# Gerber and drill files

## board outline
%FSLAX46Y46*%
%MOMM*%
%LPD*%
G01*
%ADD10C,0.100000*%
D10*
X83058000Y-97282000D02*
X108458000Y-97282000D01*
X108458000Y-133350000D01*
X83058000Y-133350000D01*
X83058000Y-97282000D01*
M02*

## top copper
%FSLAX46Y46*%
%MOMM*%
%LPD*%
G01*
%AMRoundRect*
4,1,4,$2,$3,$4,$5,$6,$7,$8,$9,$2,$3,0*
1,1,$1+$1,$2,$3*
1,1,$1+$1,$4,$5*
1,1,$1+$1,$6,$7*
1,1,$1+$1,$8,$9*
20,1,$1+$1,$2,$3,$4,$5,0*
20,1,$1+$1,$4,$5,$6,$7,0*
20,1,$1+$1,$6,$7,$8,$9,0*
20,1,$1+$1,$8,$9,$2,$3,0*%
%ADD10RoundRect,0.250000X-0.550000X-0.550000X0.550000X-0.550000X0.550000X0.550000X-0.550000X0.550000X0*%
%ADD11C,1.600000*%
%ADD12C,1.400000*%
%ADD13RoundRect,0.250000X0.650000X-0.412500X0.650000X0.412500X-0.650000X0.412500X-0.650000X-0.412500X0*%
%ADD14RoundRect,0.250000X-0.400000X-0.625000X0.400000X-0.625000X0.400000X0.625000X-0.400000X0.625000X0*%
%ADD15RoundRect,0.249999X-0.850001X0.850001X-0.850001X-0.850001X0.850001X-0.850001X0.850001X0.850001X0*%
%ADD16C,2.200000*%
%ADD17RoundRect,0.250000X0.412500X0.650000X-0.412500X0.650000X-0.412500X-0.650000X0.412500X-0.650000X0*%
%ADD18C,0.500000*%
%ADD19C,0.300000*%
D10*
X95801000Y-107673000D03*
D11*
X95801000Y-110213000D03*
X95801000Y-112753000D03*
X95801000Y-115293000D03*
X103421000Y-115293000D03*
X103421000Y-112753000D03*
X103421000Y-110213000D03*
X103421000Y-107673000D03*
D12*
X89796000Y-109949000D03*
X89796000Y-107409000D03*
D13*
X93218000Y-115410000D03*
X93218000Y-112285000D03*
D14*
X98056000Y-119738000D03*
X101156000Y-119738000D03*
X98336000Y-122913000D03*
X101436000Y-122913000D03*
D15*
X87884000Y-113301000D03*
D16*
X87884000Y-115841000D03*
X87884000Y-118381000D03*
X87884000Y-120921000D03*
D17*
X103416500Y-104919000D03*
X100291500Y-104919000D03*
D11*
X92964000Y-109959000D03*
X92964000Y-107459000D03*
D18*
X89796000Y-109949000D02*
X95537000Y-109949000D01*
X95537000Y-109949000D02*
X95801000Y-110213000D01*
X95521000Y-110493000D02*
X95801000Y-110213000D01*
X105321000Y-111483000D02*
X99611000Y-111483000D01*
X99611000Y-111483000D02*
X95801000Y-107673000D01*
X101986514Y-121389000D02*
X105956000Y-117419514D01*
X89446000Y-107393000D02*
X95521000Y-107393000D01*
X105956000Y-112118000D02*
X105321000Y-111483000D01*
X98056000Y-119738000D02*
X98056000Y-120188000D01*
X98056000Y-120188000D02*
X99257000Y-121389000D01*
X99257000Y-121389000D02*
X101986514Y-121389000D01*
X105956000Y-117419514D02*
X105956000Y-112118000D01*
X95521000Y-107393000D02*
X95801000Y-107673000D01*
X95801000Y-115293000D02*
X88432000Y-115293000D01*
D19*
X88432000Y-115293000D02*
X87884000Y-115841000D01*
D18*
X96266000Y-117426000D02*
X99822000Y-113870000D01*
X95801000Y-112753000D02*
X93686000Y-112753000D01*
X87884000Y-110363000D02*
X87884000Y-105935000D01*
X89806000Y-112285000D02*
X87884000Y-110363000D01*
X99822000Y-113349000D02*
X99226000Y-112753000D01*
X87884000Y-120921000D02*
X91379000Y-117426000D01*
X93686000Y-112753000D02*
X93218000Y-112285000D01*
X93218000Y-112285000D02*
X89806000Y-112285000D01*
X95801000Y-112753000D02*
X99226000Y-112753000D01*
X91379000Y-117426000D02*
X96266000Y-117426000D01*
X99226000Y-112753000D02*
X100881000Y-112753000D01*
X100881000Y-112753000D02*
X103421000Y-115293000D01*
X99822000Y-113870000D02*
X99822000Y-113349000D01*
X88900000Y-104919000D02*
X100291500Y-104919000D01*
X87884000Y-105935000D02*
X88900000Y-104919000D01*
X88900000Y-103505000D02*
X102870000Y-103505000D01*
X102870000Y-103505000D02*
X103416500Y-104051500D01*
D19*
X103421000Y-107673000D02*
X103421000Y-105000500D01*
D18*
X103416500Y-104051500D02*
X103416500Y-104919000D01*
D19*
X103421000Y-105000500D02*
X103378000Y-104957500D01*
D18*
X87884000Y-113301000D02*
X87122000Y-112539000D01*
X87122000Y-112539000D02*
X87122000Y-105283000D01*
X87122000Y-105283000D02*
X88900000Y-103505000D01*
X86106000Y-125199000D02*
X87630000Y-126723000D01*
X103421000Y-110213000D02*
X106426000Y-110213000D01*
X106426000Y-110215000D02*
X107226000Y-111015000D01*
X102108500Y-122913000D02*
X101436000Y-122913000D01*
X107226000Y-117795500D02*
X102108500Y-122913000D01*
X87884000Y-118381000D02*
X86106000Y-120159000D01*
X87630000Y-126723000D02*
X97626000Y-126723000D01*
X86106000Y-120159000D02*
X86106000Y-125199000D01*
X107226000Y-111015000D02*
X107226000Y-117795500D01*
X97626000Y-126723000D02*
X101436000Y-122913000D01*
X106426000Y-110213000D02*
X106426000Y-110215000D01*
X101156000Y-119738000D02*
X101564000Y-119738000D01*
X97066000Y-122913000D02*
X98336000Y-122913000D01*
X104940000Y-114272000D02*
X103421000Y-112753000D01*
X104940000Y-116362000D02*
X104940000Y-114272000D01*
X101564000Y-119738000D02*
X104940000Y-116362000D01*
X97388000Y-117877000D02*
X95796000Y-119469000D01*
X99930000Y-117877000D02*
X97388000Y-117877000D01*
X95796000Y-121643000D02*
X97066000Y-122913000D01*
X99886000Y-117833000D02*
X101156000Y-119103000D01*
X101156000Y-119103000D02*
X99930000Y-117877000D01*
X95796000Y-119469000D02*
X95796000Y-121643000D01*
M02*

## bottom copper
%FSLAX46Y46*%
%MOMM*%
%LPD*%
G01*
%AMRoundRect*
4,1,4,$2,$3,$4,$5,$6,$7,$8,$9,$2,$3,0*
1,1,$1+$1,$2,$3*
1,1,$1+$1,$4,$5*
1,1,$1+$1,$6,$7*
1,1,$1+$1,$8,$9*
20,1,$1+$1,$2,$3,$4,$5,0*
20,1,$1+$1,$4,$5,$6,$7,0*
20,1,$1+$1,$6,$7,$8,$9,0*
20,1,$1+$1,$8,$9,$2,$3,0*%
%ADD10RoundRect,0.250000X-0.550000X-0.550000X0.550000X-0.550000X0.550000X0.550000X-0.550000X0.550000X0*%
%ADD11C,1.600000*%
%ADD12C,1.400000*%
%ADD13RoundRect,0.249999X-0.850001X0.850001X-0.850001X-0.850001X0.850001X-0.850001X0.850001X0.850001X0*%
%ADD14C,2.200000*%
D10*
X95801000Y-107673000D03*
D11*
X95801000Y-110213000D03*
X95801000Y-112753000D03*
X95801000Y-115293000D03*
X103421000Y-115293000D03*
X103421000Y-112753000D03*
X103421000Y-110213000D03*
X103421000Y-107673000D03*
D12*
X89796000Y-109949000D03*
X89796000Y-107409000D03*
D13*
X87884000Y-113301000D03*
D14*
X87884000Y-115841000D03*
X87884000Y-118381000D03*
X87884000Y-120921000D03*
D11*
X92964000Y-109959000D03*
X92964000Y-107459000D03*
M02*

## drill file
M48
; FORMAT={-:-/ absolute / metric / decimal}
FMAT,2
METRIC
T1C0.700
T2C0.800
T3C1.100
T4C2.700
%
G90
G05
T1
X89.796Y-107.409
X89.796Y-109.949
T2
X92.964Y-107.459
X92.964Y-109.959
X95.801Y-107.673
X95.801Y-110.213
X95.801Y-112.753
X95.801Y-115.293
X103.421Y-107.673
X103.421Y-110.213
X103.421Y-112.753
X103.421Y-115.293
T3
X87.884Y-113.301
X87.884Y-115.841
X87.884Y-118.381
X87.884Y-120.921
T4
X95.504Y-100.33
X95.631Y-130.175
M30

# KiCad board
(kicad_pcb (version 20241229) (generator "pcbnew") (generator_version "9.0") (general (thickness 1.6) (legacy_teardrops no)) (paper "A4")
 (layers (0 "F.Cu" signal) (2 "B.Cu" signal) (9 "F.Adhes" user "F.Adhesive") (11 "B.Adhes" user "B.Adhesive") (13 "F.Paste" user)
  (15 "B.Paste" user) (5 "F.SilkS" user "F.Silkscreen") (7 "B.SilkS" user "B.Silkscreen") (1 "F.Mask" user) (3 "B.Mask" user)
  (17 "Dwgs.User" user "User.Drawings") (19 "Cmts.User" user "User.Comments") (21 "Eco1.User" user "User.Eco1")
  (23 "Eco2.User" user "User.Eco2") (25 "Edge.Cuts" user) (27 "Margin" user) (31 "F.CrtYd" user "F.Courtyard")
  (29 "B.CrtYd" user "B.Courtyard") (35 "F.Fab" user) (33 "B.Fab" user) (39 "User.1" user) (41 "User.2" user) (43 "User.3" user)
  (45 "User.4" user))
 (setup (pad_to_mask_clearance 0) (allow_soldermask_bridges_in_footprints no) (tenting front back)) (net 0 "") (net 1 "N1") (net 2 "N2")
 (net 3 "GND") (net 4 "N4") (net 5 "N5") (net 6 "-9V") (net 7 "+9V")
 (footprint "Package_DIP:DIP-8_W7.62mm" (layer "F.Cu") (at 95.801 107.673)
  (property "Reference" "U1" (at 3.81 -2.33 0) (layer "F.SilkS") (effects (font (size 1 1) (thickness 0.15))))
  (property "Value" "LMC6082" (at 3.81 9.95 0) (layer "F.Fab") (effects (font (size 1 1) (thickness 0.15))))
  (pad "1" thru_hole roundrect (at 0 0) (size 1.6 1.6) (drill 0.8) (layers "*.Cu" "*.Mask") (remove_unused_layers no)
   (roundrect_rratio 0.15625) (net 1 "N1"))
  (pad "2" thru_hole circle (at 0 2.54) (size 1.6 1.6) (drill 0.8) (layers "*.Cu" "*.Mask") (remove_unused_layers no) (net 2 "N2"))
  (pad "3" thru_hole circle (at 0 5.08) (size 1.6 1.6) (drill 0.8) (layers "*.Cu" "*.Mask") (remove_unused_layers no) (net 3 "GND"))
  (pad "4" thru_hole circle (at 0 7.62) (size 1.6 1.6) (drill 0.8) (layers "*.Cu" "*.Mask") (remove_unused_layers no))
  (pad "5" thru_hole circle (at 7.62 7.62) (size 1.6 1.6) (drill 0.8) (layers "*.Cu" "*.Mask") (remove_unused_layers no) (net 3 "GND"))
  (pad "6" thru_hole circle (at 7.62 5.08) (size 1.6 1.6) (drill 0.8) (layers "*.Cu" "*.Mask") (remove_unused_layers no) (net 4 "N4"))
  (pad "7" thru_hole circle (at 7.62 2.54) (size 1.6 1.6) (drill 0.8) (layers "*.Cu" "*.Mask") (remove_unused_layers no) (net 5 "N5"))
  (pad "8" thru_hole circle (at 7.62 0) (size 1.6 1.6) (drill 0.8) (layers "*.Cu" "*.Mask") (remove_unused_layers no)))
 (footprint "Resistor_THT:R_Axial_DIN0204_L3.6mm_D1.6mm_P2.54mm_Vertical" (layer "F.Cu") (at 89.796 109.949 90)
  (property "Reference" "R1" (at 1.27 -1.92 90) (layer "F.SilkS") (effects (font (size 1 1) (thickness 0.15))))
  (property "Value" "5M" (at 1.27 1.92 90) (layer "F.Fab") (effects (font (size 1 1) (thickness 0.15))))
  (pad "1" thru_hole circle (at 0 0 90) (size 1.4 1.4) (drill 0.7) (layers "*.Cu" "*.Mask") (remove_unused_layers no) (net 2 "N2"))
  (pad "2" thru_hole circle (at 2.54 0 90) (size 1.4 1.4) (drill 0.7) (layers "*.Cu" "*.Mask") (remove_unused_layers no) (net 1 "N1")))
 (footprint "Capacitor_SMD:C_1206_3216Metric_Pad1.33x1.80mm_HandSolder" (layer "F.Cu") (at 93.218 113.8475 90)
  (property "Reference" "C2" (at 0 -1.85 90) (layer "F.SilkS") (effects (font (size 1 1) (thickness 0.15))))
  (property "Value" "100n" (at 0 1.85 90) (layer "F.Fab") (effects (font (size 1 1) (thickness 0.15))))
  (pad "1" smd roundrect (at -1.5625 0 90) (size 1.325 1.8) (layers "F.Cu" "F.Mask" "F.Paste") (roundrect_rratio 0.188679) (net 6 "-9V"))
  (pad "2" smd roundrect (at 1.5625 0 90) (size 1.325 1.8) (layers "F.Cu" "F.Mask" "F.Paste") (roundrect_rratio 0.188679) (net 3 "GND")))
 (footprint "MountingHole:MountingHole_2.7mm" (layer "F.Cu") (at 95.631 130.175)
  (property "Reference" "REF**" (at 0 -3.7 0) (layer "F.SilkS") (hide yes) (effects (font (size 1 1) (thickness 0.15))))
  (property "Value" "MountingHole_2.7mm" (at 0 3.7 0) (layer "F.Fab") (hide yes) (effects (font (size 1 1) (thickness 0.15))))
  (pad "" np_thru_hole circle (at 0 0) (size 2.7 2.7) (drill 2.7) (layers "*.Cu" "*.Mask")))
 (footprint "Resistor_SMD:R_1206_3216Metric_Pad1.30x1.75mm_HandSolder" (layer "F.Cu") (at 99.606 119.738)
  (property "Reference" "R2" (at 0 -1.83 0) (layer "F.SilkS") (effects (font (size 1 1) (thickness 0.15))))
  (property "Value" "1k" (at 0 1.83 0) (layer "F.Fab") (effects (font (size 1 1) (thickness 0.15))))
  (pad "1" smd roundrect (at -1.55 0) (size 1.3 1.75) (layers "F.Cu" "F.Mask" "F.Paste") (roundrect_rratio 0.192308) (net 1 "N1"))
  (pad "2" smd roundrect (at 1.55 0) (size 1.3 1.75) (layers "F.Cu" "F.Mask" "F.Paste") (roundrect_rratio 0.192308) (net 4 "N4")))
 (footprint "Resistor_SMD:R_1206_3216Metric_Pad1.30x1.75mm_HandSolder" (layer "F.Cu") (at 99.886 122.913)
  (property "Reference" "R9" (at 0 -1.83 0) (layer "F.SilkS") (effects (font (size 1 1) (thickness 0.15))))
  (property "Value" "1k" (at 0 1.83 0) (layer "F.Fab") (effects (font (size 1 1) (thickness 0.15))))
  (pad "1" smd roundrect (at -1.55 0) (size 1.3 1.75) (layers "F.Cu" "F.Mask" "F.Paste") (roundrect_rratio 0.192308) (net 4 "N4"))
  (pad "2" smd roundrect (at 1.55 0) (size 1.3 1.75) (layers "F.Cu" "F.Mask" "F.Paste") (roundrect_rratio 0.192308) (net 5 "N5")))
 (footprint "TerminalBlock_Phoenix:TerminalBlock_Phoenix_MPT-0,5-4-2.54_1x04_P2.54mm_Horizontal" (layer "F.Cu") (at 87.884 113.301 -90)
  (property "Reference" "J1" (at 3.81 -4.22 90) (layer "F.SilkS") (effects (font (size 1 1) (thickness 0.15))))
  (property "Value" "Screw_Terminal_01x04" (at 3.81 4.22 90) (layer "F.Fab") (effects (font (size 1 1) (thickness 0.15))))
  (pad "1" thru_hole roundrect (at 0 0 270) (size 2.2 2.2) (drill 1.1) (layers "*.Cu" "*.Mask") (remove_unused_layers no)
   (roundrect_rratio 0.113636) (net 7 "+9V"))
  (pad "2" thru_hole circle (at 2.54 0 270) (size 2.2 2.2) (drill 1.1) (layers "*.Cu" "*.Mask") (remove_unused_layers no) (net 6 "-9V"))
  (pad "3" thru_hole circle (at 5.08 0 270) (size 2.2 2.2) (drill 1.1) (layers "*.Cu" "*.Mask") (remove_unused_layers no) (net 5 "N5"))
  (pad "4" thru_hole circle (at 7.62 0 270) (size 2.2 2.2) (drill 1.1) (layers "*.Cu" "*.Mask") (remove_unused_layers no) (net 3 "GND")))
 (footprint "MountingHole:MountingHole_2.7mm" (layer "F.Cu") (at 95.504 100.33)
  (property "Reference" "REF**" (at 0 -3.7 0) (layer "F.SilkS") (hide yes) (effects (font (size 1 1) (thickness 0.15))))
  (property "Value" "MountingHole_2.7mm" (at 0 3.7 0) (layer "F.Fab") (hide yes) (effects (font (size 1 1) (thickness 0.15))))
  (pad "" np_thru_hole circle (at 0 0) (size 2.7 2.7) (drill 2.7) (layers "*.Cu" "*.Mask")))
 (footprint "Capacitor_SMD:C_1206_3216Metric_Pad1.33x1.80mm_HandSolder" (layer "F.Cu") (at 101.854 104.919 180)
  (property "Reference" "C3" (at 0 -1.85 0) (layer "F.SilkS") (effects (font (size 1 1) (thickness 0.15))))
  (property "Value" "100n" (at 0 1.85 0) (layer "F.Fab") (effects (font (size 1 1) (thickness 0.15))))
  (pad "1" smd roundrect (at -1.5625 0 180) (size 1.325 1.8) (layers "F.Cu" "F.Mask" "F.Paste") (roundrect_rratio 0.188679) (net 7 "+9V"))
  (pad "2" smd roundrect (at 1.5625 0 180) (size 1.325 1.8) (layers "F.Cu" "F.Mask" "F.Paste") (roundrect_rratio 0.188679) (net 3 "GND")))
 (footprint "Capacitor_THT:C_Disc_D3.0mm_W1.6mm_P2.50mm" (layer "F.Cu") (at 92.964 109.959 90)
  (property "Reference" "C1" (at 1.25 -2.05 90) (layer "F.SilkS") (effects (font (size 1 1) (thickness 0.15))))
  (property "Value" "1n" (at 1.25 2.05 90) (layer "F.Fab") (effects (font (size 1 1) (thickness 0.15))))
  (pad "1" thru_hole circle (at 0 0 90) (size 1.6 1.6) (drill 0.8) (layers "*.Cu" "*.Mask") (remove_unused_layers no) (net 2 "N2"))
  (pad "2" thru_hole circle (at 2.5 0 90) (size 1.6 1.6) (drill 0.8) (layers "*.Cu" "*.Mask") (remove_unused_layers no) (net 1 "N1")))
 (gr_rect (start 83.058 97.282) (end 108.458 133.35) (stroke (width 0.1) (type solid)) (fill no) (layer "Edge.Cuts"))
 (segment (start 89.796 109.949) (end 95.537 109.949) (width 0.5) (layer "F.Cu") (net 2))
 (segment (start 95.537 109.949) (end 95.801 110.213) (width 0.5) (layer "F.Cu") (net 2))
 (segment (start 95.521 110.493) (end 95.801 110.213) (width 0.5) (layer "F.Cu") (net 2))
 (segment (start 105.321 111.483) (end 99.611 111.483) (width 0.5) (layer "F.Cu") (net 1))
 (segment (start 99.611 111.483) (end 95.801 107.673) (width 0.5) (layer "F.Cu") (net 1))
 (segment (start 101.986514 121.389) (end 105.956 117.419514) (width 0.5) (layer "F.Cu") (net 1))
 (segment (start 89.446 107.393) (end 95.521 107.393) (width 0.5) (layer "F.Cu") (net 1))
 (segment (start 105.956 112.118) (end 105.321 111.483) (width 0.5) (layer "F.Cu") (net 1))
 (segment (start 98.056 119.738) (end 98.056 120.188) (width 0.5) (layer "F.Cu") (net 1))
 (segment (start 98.056 120.188) (end 99.257 121.389) (width 0.5) (layer "F.Cu") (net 1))
 (segment (start 99.257 121.389) (end 101.986514 121.389) (width 0.5) (layer "F.Cu") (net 1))
 (segment (start 105.956 117.419514) (end 105.956 112.118) (width 0.5) (layer "F.Cu") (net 1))
 (segment (start 95.521 107.393) (end 95.801 107.673) (width 0.5) (layer "F.Cu") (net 1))
 (segment (start 95.801 115.293) (end 88.432 115.293) (width 0.5) (layer "F.Cu") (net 6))
 (segment (start 88.432 115.293) (end 87.884 115.841) (width 0.3) (layer "F.Cu") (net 6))
 (segment (start 96.266 117.426) (end 99.822 113.87) (width 0.5) (layer "F.Cu") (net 3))
 (segment (start 95.801 112.753) (end 93.686 112.753) (width 0.5) (layer "F.Cu") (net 3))
 (segment (start 87.884 110.363) (end 87.884 105.935) (width 0.5) (layer "F.Cu") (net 3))
 (segment (start 89.806 112.285) (end 87.884 110.363) (width 0.5) (layer "F.Cu") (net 3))
 (segment (start 99.822 113.349) (end 99.226 112.753) (width 0.5) (layer "F.Cu") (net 3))
 (segment (start 87.884 120.921) (end 91.379 117.426) (width 0.5) (layer "F.Cu") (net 3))
 (segment (start 93.686 112.753) (end 93.218 112.285) (width 0.5) (layer "F.Cu") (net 3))
 (segment (start 93.218 112.285) (end 89.806 112.285) (width 0.5) (layer "F.Cu") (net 3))
 (segment (start 95.801 112.753) (end 99.226 112.753) (width 0.5) (layer "F.Cu") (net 3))
 (segment (start 91.379 117.426) (end 96.266 117.426) (width 0.5) (layer "F.Cu") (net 3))
 (segment (start 99.226 112.753) (end 100.881 112.753) (width 0.5) (layer "F.Cu") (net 3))
 (segment (start 100.881 112.753) (end 103.421 115.293) (width 0.5) (layer "F.Cu") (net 3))
 (segment (start 99.822 113.87) (end 99.822 113.349) (width 0.5) (layer "F.Cu") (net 3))
 (segment (start 88.9 104.919) (end 100.2915 104.919) (width 0.5) (layer "F.Cu") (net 3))
 (segment (start 87.884 105.935) (end 88.9 104.919) (width 0.5) (layer "F.Cu") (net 3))
 (segment (start 88.9 103.505) (end 102.87 103.505) (width 0.5) (layer "F.Cu") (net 7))
 (segment (start 102.87 103.505) (end 103.4165 104.0515) (width 0.5) (layer "F.Cu") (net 7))
 (segment (start 103.421 107.673) (end 103.421 105.0005) (width 0.3) (layer "F.Cu") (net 7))
 (segment (start 103.4165 104.0515) (end 103.4165 104.919) (width 0.5) (layer "F.Cu") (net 7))
 (segment (start 103.421 105.0005) (end 103.378 104.9575) (width 0.3) (layer "F.Cu") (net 7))
 (segment (start 87.884 113.301) (end 87.122 112.539) (width 0.5) (layer "F.Cu") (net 7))
 (segment (start 87.122 112.539) (end 87.122 105.283) (width 0.5) (layer "F.Cu") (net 7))
 (segment (start 87.122 105.283) (end 88.9 103.505) (width 0.5) (layer "F.Cu") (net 7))
 (segment (start 86.106 125.199) (end 87.63 126.723) (width 0.5) (layer "F.Cu") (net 5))
 (segment (start 103.421 110.213) (end 106.426 110.213) (width 0.5) (layer "F.Cu") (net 5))
 (segment (start 106.426 110.215) (end 107.226 111.015) (width 0.5) (layer "F.Cu") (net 5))
 (segment (start 102.1085 122.913) (end 101.436 122.913) (width 0.5) (layer "F.Cu") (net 5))
 (segment (start 107.226 117.7955) (end 102.1085 122.913) (width 0.5) (layer "F.Cu") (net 5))
 (segment (start 87.884 118.381) (end 86.106 120.159) (width 0.5) (layer "F.Cu") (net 5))
 (segment (start 87.63 126.723) (end 97.626 126.723) (width 0.5) (layer "F.Cu") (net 5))
 (segment (start 86.106 120.159) (end 86.106 125.199) (width 0.5) (layer "F.Cu") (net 5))
 (segment (start 107.226 111.015) (end 107.226 117.7955) (width 0.5) (layer "F.Cu") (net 5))
 (segment (start 97.626 126.723) (end 101.436 122.913) (width 0.5) (layer "F.Cu") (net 5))
 (segment (start 106.426 110.213) (end 106.426 110.215) (width 0.5) (layer "F.Cu") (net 5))
 (segment (start 101.156 119.738) (end 101.564 119.738) (width 0.5) (layer "F.Cu") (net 4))
 (segment (start 97.066 122.913) (end 98.336 122.913) (width 0.5) (layer "F.Cu") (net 4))
 (segment (start 104.94 114.272) (end 103.421 112.753) (width 0.5) (layer "F.Cu") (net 4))
 (segment (start 104.94 116.362) (end 104.94 114.272) (width 0.5) (layer "F.Cu") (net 4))
 (segment (start 101.564 119.738) (end 104.94 116.362) (width 0.5) (layer "F.Cu") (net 4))
 (segment (start 97.388 117.877) (end 95.796 119.469) (width 0.5) (layer "F.Cu") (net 4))
 (segment (start 99.93 117.877) (end 97.388 117.877) (width 0.5) (layer "F.Cu") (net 4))
 (segment (start 95.796 121.643) (end 97.066 122.913) (width 0.5) (layer "F.Cu") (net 4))
 (segment (start 99.886 117.833) (end 101.156 119.103) (width 0.5) (layer "F.Cu") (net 4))
 (segment (start 101.156 119.103) (end 99.93 117.877) (width 0.5) (layer "F.Cu") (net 4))
 (segment (start 95.796 119.469) (end 95.796 121.643) (width 0.5) (layer "F.Cu") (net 4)))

